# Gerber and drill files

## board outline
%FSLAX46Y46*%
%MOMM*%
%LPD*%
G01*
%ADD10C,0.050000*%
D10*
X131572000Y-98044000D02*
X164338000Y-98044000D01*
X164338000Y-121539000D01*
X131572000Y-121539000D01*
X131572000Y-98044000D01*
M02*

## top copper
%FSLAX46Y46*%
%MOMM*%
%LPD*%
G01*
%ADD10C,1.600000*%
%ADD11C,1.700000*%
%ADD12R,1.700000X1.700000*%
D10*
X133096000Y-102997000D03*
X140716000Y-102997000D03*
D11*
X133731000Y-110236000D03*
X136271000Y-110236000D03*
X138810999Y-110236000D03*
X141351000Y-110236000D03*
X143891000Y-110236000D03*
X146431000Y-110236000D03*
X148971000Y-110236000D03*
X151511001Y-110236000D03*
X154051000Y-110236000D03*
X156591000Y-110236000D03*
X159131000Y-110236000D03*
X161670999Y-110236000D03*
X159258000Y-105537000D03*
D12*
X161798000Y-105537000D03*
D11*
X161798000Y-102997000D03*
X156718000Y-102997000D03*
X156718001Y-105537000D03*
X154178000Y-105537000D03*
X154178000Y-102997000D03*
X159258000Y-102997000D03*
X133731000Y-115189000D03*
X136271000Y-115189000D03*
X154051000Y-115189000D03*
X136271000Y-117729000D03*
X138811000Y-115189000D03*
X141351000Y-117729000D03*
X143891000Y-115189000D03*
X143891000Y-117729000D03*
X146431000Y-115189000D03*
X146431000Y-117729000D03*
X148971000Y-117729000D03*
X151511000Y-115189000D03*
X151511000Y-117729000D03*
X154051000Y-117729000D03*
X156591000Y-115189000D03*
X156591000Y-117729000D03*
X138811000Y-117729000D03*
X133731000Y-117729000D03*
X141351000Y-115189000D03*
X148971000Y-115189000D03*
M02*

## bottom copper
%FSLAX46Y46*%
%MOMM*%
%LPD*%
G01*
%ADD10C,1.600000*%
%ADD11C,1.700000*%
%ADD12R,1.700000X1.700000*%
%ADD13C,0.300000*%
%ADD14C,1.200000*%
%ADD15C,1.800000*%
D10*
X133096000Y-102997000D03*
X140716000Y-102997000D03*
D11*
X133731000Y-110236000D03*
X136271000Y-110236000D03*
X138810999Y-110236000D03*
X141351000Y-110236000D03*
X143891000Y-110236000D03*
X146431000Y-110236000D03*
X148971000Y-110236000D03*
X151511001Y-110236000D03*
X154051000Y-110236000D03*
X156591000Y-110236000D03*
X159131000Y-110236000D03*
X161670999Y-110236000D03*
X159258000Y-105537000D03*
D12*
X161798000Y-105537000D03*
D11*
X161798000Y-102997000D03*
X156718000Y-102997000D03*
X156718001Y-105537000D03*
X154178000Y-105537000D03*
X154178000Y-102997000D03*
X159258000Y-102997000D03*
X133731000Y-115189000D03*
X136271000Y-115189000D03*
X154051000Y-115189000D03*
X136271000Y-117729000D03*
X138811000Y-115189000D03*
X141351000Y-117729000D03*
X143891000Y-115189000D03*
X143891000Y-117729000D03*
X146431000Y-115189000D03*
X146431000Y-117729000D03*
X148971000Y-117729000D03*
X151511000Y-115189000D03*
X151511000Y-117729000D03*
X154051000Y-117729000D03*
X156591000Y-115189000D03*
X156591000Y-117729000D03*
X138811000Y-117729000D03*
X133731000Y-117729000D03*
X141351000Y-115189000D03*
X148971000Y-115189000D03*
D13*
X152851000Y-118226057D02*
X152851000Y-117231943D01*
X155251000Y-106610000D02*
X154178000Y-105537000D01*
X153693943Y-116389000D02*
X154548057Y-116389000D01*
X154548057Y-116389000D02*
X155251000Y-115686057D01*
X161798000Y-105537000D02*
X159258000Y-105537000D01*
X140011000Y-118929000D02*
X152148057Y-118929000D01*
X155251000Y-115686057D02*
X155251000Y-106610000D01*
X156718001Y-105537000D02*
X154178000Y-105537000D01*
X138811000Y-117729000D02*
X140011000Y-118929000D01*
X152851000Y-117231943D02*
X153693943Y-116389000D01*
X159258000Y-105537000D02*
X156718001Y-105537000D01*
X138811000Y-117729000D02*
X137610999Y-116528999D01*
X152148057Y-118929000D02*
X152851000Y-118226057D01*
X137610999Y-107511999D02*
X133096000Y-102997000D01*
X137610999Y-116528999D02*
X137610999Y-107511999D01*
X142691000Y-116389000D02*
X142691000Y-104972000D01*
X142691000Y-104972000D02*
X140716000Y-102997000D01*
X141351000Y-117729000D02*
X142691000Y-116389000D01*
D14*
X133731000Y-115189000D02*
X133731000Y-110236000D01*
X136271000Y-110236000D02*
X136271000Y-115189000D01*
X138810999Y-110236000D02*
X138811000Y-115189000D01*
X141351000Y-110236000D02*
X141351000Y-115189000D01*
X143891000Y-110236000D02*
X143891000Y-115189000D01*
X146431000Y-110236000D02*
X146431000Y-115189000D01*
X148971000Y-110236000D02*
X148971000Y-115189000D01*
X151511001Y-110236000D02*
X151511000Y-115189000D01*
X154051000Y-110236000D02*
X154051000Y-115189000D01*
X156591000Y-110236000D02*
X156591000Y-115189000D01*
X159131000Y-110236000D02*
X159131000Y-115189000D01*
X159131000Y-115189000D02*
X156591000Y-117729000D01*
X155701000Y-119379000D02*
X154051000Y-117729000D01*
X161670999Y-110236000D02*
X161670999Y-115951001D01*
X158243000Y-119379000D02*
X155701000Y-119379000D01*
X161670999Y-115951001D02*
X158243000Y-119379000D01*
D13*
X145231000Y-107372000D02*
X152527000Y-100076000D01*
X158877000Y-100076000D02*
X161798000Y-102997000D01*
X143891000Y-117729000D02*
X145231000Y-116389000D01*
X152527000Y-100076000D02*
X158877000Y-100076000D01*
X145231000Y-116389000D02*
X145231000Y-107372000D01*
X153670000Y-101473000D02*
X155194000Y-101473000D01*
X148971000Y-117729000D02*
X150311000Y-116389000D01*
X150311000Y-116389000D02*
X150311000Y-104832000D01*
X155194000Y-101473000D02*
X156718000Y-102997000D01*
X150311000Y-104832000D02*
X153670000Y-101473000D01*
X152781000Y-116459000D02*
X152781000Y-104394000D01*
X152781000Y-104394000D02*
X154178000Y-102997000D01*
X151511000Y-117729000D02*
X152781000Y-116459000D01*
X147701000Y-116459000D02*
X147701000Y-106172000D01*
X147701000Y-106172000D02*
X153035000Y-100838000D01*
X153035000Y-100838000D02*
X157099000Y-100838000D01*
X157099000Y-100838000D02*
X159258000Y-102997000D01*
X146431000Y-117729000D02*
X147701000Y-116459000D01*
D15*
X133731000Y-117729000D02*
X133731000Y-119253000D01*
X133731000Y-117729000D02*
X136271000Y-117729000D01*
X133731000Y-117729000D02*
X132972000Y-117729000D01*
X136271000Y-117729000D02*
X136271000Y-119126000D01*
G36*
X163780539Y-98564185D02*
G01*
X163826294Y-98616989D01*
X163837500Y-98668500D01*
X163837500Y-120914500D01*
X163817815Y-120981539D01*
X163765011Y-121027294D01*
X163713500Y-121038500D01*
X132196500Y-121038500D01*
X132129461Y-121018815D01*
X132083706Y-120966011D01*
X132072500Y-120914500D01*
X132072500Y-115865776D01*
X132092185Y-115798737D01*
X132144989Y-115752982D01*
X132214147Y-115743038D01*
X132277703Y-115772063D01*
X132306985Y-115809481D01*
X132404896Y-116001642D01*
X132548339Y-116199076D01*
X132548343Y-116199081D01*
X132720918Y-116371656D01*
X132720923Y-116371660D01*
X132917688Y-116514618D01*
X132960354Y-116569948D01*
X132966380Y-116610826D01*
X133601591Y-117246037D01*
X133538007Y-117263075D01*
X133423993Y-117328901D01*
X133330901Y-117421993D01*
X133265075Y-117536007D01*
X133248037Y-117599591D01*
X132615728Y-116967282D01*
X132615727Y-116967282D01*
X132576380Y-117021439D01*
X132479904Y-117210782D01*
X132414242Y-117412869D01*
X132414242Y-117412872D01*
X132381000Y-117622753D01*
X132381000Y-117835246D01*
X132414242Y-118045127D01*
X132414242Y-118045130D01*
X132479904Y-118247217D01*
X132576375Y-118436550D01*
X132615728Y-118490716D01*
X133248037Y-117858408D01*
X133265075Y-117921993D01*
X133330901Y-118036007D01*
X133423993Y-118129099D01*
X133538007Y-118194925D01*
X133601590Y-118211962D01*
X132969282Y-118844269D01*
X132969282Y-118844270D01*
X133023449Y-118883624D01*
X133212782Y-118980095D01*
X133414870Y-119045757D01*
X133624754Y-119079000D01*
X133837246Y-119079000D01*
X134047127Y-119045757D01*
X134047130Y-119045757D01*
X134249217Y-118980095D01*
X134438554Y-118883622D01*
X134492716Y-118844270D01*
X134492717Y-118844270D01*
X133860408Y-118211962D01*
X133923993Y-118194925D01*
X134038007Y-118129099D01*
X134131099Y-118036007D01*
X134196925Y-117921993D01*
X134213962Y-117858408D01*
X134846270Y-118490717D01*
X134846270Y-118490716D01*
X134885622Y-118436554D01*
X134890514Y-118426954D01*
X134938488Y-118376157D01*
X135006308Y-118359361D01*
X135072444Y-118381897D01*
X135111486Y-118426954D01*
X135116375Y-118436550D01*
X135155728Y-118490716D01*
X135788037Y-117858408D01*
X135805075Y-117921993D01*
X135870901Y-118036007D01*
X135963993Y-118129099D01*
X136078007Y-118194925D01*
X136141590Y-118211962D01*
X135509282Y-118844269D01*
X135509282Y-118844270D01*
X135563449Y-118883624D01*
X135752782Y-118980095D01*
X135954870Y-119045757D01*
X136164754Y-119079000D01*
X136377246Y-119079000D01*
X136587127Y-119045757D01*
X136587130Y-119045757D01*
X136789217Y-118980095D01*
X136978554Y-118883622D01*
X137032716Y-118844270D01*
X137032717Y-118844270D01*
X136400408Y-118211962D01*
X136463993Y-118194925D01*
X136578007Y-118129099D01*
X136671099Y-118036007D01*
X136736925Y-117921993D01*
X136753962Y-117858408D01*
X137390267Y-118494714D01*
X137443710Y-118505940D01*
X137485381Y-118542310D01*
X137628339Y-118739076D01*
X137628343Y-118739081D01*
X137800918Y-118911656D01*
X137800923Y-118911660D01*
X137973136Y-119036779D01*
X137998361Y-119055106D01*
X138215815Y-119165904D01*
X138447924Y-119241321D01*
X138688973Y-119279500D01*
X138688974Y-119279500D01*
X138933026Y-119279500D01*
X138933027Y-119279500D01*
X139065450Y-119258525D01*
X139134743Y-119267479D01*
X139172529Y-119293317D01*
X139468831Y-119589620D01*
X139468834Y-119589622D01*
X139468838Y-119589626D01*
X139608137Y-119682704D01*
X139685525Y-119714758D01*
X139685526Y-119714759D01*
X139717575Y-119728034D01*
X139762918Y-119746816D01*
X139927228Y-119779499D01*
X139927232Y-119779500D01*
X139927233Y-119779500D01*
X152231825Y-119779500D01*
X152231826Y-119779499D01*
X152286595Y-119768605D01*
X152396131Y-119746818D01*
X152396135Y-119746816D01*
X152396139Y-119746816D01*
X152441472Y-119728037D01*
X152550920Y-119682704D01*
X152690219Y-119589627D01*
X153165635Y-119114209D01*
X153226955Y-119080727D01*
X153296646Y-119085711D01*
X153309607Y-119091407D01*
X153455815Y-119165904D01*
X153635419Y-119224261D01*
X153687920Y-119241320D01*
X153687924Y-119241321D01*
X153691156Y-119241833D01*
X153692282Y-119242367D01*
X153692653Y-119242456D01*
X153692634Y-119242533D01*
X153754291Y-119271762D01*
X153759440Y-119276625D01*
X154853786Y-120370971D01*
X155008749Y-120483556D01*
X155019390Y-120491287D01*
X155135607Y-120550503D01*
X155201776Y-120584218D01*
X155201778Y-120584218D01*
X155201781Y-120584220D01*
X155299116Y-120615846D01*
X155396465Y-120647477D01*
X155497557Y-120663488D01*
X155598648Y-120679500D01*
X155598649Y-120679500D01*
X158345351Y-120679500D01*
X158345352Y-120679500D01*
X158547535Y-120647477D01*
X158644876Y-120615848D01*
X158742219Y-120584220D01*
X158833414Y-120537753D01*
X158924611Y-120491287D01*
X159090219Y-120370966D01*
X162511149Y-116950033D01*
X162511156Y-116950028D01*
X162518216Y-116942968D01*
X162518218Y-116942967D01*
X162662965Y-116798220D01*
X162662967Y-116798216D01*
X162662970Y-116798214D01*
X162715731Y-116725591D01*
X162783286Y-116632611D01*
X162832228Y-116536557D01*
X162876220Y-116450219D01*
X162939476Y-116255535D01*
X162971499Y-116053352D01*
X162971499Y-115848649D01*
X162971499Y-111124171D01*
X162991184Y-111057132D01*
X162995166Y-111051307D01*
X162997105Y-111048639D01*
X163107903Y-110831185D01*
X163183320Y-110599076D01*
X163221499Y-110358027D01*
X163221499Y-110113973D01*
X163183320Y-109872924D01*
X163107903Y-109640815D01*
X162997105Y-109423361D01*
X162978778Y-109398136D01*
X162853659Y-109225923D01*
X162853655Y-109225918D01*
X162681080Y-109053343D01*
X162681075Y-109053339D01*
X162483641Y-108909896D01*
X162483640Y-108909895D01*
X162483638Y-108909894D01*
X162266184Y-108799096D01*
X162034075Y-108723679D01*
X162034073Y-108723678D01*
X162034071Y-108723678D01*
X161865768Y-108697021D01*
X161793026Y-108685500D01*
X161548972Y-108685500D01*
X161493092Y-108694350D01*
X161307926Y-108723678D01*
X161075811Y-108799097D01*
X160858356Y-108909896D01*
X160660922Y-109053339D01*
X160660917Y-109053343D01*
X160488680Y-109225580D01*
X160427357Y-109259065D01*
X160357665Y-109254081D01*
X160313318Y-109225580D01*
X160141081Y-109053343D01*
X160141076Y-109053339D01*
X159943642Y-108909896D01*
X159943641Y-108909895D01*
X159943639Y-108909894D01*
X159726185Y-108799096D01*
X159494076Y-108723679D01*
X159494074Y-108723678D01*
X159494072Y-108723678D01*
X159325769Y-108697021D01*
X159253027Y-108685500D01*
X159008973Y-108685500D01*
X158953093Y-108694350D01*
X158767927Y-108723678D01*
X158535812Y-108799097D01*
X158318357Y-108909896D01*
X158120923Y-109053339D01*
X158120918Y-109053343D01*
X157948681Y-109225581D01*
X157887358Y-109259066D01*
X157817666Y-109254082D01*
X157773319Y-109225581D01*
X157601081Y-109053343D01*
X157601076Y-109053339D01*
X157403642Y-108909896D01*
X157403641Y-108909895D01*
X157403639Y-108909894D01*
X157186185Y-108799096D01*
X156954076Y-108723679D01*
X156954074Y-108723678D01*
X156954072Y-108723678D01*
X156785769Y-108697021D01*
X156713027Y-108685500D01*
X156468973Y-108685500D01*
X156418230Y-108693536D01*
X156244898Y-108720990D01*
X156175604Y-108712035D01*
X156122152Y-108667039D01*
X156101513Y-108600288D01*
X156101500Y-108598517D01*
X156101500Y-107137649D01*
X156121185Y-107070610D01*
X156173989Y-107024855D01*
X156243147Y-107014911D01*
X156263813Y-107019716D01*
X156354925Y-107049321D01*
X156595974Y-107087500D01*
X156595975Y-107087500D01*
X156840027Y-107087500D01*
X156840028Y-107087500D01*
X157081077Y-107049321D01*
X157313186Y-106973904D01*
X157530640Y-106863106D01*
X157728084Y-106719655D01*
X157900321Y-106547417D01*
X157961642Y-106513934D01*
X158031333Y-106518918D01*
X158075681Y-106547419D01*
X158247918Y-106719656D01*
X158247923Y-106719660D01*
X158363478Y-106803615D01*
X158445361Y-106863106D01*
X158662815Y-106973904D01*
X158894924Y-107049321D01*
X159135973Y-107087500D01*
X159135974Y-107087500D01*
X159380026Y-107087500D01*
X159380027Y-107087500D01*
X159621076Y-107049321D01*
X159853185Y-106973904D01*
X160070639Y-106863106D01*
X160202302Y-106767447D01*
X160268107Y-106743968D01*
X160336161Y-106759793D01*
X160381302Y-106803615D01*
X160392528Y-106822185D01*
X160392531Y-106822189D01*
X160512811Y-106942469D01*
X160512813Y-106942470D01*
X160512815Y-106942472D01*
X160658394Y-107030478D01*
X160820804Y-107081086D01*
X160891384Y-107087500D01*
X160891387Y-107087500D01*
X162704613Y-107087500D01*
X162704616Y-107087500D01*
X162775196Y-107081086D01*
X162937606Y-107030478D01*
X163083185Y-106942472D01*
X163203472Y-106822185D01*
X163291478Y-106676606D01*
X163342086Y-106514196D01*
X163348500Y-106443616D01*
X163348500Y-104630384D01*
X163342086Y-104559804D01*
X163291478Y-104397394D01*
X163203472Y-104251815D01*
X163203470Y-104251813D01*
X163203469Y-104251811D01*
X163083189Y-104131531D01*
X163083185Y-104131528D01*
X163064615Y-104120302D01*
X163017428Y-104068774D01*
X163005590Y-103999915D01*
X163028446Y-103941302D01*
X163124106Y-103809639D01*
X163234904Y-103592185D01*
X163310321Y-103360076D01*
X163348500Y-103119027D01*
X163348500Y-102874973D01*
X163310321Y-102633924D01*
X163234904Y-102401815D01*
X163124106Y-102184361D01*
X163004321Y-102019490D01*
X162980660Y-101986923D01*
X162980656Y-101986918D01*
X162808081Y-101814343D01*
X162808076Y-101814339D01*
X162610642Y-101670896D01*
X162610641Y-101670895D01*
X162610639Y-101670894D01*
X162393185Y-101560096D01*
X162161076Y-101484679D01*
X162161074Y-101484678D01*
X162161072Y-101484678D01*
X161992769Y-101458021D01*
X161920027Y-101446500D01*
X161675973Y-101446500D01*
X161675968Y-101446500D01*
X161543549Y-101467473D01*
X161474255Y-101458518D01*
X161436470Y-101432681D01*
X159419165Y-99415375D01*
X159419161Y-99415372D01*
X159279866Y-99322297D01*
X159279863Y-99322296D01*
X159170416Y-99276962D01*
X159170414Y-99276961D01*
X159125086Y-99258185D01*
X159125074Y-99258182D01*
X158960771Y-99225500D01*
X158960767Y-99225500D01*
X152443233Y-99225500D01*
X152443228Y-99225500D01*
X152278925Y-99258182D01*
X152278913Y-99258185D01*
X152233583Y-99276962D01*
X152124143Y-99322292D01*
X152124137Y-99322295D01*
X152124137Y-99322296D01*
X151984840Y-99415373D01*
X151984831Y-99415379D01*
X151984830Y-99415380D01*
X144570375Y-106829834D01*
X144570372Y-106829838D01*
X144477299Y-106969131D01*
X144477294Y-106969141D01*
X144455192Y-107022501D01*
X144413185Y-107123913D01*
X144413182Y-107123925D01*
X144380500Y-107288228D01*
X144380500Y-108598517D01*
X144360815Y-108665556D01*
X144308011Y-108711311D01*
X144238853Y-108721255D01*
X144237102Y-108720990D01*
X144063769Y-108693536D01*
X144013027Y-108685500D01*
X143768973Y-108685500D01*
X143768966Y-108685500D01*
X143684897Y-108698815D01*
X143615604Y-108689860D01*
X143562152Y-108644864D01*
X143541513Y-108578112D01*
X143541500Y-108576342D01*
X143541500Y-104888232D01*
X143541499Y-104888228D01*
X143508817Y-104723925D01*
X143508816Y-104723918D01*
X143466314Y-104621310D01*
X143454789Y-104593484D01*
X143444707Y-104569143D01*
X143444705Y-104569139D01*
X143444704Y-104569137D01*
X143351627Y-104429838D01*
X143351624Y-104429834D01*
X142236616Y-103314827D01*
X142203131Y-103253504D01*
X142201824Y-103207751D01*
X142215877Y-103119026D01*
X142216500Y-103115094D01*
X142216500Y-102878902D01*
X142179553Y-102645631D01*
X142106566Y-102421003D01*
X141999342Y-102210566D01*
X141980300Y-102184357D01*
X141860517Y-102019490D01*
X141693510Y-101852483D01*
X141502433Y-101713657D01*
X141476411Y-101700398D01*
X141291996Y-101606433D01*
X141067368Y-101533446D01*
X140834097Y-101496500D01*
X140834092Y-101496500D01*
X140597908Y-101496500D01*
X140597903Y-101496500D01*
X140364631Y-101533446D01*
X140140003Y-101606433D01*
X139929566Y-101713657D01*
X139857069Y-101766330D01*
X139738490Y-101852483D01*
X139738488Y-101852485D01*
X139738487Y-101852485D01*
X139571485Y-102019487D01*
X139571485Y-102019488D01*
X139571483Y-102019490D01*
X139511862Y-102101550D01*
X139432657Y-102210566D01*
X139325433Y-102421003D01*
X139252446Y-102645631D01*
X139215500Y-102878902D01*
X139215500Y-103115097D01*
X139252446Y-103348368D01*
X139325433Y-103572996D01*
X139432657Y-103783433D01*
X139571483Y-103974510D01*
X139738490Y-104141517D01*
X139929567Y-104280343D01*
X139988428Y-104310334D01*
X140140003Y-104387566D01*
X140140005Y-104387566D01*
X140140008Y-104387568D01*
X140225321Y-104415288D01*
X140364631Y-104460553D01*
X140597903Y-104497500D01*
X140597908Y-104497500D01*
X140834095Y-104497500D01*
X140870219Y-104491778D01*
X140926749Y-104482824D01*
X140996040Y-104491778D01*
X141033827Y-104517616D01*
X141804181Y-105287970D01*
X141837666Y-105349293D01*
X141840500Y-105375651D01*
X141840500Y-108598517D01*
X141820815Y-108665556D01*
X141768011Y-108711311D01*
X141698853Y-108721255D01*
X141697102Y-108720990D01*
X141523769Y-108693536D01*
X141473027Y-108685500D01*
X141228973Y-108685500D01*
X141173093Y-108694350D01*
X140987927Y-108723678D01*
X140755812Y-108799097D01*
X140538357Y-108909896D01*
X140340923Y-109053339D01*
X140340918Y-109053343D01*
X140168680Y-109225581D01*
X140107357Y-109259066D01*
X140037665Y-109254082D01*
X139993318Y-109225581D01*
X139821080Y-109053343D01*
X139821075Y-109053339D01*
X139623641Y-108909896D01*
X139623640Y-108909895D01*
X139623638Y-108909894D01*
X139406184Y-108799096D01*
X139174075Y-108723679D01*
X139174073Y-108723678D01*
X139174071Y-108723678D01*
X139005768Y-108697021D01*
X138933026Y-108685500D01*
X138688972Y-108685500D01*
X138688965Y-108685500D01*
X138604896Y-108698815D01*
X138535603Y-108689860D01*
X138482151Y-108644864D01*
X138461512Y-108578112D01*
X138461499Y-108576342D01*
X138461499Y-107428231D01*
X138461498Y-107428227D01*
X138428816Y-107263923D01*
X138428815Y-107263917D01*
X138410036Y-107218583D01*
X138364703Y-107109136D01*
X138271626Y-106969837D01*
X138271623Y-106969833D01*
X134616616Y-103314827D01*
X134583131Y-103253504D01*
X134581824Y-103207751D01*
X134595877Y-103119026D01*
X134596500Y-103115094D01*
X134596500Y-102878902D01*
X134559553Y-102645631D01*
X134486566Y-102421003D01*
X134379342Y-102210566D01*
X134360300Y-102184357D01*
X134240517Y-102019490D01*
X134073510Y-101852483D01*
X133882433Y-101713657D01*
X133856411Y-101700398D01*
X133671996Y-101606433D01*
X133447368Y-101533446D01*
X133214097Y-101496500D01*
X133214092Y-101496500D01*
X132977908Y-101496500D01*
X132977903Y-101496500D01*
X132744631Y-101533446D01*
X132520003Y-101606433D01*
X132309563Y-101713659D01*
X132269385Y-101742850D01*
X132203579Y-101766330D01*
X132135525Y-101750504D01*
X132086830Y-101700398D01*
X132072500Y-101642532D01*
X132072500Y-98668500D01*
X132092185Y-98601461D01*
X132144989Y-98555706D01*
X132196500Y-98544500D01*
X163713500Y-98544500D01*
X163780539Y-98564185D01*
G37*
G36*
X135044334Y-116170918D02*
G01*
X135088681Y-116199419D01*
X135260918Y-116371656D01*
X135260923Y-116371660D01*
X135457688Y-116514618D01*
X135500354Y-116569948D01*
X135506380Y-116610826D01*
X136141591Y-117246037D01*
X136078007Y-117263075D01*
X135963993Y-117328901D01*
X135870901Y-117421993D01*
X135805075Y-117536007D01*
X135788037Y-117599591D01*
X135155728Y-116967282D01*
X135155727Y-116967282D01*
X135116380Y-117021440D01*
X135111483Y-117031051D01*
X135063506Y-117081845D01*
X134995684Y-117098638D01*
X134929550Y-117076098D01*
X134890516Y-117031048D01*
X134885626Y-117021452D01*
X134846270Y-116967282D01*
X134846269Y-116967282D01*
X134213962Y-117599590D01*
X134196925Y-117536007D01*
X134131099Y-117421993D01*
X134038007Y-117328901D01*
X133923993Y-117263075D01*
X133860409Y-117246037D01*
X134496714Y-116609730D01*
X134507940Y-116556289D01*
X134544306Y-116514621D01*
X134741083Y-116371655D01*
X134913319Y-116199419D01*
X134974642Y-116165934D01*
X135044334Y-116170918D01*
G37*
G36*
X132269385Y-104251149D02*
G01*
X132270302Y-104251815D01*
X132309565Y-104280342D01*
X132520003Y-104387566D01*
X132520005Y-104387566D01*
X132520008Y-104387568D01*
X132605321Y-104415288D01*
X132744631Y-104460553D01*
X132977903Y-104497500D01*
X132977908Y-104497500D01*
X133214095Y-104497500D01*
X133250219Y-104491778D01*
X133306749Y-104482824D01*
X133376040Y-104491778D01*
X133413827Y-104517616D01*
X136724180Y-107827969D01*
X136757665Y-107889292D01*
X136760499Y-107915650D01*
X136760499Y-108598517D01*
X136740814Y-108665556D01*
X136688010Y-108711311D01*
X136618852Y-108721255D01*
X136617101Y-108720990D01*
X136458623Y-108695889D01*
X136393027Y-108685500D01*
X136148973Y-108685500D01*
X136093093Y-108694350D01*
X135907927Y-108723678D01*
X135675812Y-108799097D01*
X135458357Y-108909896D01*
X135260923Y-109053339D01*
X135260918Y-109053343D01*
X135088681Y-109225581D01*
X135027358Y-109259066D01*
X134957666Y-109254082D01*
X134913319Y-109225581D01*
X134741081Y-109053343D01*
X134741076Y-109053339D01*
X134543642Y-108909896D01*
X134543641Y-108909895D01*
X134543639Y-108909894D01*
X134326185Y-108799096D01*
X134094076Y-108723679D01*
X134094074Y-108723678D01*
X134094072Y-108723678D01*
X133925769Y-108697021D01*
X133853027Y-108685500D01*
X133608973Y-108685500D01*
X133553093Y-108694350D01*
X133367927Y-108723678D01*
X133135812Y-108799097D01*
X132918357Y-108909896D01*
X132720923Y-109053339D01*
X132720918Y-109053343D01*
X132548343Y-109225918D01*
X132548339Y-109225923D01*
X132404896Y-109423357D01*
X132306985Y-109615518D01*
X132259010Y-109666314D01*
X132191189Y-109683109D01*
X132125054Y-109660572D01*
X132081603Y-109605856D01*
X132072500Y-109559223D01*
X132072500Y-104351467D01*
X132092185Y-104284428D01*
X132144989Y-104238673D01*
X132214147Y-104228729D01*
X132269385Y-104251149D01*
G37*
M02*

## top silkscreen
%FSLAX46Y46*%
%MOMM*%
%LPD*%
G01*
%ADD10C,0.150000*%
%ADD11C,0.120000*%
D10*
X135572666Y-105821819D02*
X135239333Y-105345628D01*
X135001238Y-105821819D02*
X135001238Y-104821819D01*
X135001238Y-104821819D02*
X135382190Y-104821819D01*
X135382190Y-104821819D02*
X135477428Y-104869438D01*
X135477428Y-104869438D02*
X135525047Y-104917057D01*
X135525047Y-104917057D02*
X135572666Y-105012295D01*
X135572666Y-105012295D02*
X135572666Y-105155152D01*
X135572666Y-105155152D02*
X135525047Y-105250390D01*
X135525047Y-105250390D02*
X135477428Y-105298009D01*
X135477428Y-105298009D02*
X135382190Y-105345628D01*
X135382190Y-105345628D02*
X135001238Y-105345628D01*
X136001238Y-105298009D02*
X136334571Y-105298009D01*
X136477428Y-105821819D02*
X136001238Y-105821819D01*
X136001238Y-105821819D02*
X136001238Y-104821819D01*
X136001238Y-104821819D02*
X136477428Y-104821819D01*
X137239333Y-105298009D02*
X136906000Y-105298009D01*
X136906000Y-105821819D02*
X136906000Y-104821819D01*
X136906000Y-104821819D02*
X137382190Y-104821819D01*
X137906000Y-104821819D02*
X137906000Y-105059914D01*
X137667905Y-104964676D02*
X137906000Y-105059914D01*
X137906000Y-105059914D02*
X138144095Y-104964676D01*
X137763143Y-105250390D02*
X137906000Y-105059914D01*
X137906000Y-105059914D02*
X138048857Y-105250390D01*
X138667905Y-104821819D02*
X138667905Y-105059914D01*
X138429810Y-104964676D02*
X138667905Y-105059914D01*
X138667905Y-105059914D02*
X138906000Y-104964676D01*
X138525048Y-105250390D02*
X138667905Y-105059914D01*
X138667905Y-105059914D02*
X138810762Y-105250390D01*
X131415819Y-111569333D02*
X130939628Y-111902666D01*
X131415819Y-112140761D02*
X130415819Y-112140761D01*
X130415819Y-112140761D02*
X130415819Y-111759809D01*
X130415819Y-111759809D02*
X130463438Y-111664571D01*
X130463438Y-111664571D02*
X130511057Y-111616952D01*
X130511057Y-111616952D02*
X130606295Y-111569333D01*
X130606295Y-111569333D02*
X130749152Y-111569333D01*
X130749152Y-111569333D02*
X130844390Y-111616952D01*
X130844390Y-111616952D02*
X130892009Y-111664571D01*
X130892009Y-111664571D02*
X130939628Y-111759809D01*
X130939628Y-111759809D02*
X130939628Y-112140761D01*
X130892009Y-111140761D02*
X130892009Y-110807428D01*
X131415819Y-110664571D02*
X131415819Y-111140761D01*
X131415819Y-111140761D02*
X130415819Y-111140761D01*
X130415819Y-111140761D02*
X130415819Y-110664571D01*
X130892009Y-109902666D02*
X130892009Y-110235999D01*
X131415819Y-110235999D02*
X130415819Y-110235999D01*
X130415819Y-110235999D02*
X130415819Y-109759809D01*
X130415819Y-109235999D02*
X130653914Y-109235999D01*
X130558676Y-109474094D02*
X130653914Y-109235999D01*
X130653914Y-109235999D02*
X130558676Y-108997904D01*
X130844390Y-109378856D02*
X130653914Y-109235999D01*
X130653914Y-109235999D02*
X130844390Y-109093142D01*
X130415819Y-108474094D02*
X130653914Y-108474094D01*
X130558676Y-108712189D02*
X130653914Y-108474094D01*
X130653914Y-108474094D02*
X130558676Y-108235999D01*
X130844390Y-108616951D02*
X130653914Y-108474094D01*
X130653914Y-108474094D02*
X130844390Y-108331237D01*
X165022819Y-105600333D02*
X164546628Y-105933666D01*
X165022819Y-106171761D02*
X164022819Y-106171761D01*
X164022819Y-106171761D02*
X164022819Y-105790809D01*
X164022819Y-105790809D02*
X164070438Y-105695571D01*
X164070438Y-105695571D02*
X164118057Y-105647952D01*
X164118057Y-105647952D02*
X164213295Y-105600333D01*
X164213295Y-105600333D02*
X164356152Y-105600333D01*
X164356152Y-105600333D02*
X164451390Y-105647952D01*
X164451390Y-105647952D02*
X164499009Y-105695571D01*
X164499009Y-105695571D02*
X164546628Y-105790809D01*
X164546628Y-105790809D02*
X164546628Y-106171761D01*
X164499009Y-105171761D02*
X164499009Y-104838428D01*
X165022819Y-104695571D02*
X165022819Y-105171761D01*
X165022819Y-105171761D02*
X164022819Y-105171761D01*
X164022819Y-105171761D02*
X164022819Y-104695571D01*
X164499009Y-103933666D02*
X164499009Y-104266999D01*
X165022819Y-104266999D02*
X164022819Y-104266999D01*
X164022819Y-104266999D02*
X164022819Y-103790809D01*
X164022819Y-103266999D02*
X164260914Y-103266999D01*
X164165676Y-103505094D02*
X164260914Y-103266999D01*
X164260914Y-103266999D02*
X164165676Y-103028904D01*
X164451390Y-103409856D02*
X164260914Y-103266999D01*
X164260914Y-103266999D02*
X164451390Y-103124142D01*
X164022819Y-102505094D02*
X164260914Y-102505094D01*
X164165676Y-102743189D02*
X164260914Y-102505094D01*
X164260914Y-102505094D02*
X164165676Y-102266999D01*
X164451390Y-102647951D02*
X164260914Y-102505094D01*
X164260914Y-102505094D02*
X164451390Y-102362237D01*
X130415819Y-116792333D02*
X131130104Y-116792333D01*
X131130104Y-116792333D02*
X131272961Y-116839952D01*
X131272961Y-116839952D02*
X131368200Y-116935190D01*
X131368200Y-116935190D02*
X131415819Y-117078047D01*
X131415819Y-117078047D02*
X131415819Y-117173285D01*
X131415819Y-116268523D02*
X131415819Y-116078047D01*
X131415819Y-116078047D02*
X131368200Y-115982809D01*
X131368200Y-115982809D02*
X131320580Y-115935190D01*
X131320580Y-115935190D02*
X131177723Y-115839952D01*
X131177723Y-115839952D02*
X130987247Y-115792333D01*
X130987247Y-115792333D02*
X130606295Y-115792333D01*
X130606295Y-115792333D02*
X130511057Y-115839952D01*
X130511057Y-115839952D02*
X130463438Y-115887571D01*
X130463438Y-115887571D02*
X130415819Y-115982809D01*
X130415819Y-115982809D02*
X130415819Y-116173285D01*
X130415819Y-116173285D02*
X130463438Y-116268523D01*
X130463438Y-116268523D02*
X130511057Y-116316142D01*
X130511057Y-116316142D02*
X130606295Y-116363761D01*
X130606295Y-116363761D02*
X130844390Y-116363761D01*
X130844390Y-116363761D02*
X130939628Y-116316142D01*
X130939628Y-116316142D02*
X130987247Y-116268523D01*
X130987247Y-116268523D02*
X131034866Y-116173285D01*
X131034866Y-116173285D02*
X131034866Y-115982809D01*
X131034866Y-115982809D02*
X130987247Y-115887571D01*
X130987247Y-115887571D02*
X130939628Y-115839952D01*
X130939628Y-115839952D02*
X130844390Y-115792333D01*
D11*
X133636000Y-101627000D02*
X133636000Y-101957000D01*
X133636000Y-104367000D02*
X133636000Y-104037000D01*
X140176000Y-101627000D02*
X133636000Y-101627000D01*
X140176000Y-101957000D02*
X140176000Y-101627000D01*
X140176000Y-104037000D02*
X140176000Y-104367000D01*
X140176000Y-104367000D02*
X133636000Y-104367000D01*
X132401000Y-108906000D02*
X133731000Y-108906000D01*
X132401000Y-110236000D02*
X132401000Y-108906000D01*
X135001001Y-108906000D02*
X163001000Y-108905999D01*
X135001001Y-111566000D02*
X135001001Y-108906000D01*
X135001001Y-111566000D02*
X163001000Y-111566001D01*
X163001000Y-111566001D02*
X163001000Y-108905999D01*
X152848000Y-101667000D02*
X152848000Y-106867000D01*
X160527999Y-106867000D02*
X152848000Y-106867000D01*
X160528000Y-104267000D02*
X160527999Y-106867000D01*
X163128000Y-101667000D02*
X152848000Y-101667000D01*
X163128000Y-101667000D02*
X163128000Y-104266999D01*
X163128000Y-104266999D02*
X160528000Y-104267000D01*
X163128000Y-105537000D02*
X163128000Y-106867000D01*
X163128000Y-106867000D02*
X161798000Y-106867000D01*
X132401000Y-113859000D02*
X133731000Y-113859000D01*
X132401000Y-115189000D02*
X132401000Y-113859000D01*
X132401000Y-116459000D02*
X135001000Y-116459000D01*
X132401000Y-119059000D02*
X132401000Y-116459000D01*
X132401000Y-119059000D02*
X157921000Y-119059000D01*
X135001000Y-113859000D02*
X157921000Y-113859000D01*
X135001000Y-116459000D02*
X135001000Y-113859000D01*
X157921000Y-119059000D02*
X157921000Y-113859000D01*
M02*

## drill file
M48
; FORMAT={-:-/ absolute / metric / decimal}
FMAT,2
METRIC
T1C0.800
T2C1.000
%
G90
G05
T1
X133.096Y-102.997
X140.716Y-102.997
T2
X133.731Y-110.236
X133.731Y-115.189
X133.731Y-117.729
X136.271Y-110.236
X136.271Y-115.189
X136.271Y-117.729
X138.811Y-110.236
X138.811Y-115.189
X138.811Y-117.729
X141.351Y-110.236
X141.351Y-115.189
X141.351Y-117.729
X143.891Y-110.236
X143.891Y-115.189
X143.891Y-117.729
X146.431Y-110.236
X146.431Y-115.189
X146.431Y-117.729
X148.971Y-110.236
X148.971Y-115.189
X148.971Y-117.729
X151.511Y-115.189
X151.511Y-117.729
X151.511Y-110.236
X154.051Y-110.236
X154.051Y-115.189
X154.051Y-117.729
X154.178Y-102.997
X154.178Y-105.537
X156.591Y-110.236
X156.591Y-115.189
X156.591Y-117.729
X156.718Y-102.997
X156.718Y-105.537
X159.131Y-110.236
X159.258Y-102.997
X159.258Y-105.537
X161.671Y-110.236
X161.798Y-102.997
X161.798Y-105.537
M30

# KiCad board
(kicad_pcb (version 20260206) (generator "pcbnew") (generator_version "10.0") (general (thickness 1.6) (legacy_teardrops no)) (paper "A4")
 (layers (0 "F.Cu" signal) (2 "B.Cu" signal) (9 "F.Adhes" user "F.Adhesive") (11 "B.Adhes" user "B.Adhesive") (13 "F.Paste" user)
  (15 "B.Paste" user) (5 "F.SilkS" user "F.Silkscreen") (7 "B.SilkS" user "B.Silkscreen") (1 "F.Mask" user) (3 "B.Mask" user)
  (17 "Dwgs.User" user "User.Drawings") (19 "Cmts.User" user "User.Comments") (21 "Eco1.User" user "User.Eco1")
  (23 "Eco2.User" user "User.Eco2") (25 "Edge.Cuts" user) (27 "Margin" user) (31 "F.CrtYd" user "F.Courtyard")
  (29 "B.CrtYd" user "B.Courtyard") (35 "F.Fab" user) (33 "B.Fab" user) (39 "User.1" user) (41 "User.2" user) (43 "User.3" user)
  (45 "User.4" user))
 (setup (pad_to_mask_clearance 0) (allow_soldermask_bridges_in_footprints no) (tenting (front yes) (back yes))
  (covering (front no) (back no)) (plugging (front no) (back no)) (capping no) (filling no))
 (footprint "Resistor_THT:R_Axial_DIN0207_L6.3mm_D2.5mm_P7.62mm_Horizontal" (layer "F.Cu") (at 140.716 102.997 180)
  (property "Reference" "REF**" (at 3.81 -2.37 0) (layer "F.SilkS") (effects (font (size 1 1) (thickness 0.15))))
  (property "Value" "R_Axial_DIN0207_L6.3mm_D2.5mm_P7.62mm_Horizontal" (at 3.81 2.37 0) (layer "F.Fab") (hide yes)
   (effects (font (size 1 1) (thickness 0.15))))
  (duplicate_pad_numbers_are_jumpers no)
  (fp_line (start 7.08 1.37) (end 7.08 1.04) (stroke (width 0.12) (type solid)) (layer "F.SilkS"))
  (fp_line (start 7.08 -1.37) (end 7.08 -1.04) (stroke (width 0.12) (type solid)) (layer "F.SilkS"))
  (fp_line (start 0.54 1.37) (end 7.08 1.37) (stroke (width 0.12) (type solid)) (layer "F.SilkS"))
  (fp_line (start 0.54 1.04) (end 0.54 1.37) (stroke (width 0.12) (type solid)) (layer "F.SilkS"))
  (fp_line (start 0.54 -1.04) (end 0.54 -1.37) (stroke (width 0.12) (type solid)) (layer "F.SilkS"))
  (fp_line (start 0.54 -1.37) (end 7.08 -1.37) (stroke (width 0.12) (type solid)) (layer "F.SilkS"))
  (pad "3" thru_hole circle (at 7.62 0 180) (size 1.6 1.6) (drill 0.8) (layers "*.Cu" "*.Mask") (remove_unused_layers no) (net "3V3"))
  (pad "con" thru_hole circle (at 0 0 180) (size 1.6 1.6) (drill 0.8) (layers "*.Cu" "*.Mask") (remove_unused_layers no) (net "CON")))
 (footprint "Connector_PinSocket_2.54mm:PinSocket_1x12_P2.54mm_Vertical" (layer "F.Cu") (at 133.731 110.236 90)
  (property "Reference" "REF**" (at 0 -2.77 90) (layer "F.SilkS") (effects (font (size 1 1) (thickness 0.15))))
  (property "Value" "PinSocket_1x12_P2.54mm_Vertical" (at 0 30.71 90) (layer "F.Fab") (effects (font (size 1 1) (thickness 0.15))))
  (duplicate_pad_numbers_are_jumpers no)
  (fp_line (start 1.33 -1.33) (end 1.33 0) (stroke (width 0.12) (type solid)) (layer "F.SilkS"))
  (fp_line (start 0 -1.33) (end 1.33 -1.33) (stroke (width 0.12) (type solid)) (layer "F.SilkS"))
  (fp_line (start 1.33 1.270001) (end 1.330001 29.27) (stroke (width 0.12) (type solid)) (layer "F.SilkS"))
  (fp_line (start -1.33 1.270001) (end 1.33 1.270001) (stroke (width 0.12) (type solid)) (layer "F.SilkS"))
  (fp_line (start -1.33 1.270001) (end -1.330001 29.27) (stroke (width 0.12) (type solid)) (layer "F.SilkS"))
  (fp_line (start -1.330001 29.27) (end 1.330001 29.27) (stroke (width 0.12) (type solid)) (layer "F.SilkS"))
  (pad "1" thru_hole circle (at 0 0 90) (size 1.7 1.7) (drill 1) (layers "*.Cu" "*.Mask") (remove_unused_layers no) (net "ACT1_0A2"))
  (pad "2" thru_hole circle (at 0 2.54 90) (size 1.7 1.7) (drill 1) (layers "*.Cu" "*.Mask") (remove_unused_layers no) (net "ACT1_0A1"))
  (pad "3" thru_hole circle (at 0 5.079999 90) (size 1.7 1.7) (drill 1) (layers "*.Cu" "*.Mask") (remove_unused_layers no) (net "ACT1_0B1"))
  (pad "4" thru_hole circle (at 0 7.62 90) (size 1.7 1.7) (drill 1) (layers "*.Cu" "*.Mask") (remove_unused_layers no) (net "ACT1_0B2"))
  (pad "5" thru_hole circle (at 0 10.16 90) (size 1.7 1.7) (drill 1) (layers "*.Cu" "*.Mask") (remove_unused_layers no) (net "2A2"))
  (pad "6" thru_hole circle (at 0 12.7 90) (size 1.7 1.7) (drill 1) (layers "*.Cu" "*.Mask") (remove_unused_layers no) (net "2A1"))
  (pad "7" thru_hole circle (at 0 15.24 90) (size 1.7 1.7) (drill 1) (layers "*.Cu" "*.Mask") (remove_unused_layers no) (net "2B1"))
  (pad "8" thru_hole circle (at 0 17.780001 90) (size 1.7 1.7) (drill 1) (layers "*.Cu" "*.Mask") (remove_unused_layers no) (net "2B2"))
  (pad "9" thru_hole circle (at 0 20.32 90) (size 1.7 1.7) (drill 1) (layers "*.Cu" "*.Mask") (remove_unused_layers no) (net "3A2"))
  (pad "10" thru_hole circle (at 0 22.86 90) (size 1.7 1.7) (drill 1) (layers "*.Cu" "*.Mask") (remove_unused_layers no) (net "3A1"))
  (pad "11" thru_hole circle (at 0 25.4 90) (size 1.7 1.7) (drill 1) (layers "*.Cu" "*.Mask") (remove_unused_layers no) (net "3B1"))
  (pad "12" thru_hole circle (at 0 27.939999 90) (size 1.7 1.7) (drill 1) (layers "*.Cu" "*.Mask") (remove_unused_layers no) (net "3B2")))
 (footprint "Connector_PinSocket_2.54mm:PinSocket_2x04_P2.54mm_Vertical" (layer "F.Cu") (at 161.798 105.537 -90)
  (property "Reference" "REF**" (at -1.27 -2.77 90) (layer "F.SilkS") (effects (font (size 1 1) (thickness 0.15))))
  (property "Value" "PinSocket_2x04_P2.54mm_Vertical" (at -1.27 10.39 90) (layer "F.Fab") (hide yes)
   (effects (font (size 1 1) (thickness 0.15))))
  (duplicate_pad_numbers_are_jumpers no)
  (fp_line (start -3.87 8.95) (end 1.33 8.95) (stroke (width 0.12) (type solid)) (layer "F.SilkS"))
  (fp_line (start 1.33 1.270001) (end 1.33 8.95) (stroke (width 0.12) (type solid)) (layer "F.SilkS"))
  (fp_line (start -1.27 1.27) (end 1.33 1.270001) (stroke (width 0.12) (type solid)) (layer "F.SilkS"))
  (fp_line (start -3.87 -1.33) (end -3.87 8.95) (stroke (width 0.12) (type solid)) (layer "F.SilkS"))
  (fp_line (start -3.87 -1.33) (end -1.270001 -1.33) (stroke (width 0.12) (type solid)) (layer "F.SilkS"))
  (fp_line (start -1.270001 -1.33) (end -1.27 1.27) (stroke (width 0.12) (type solid)) (layer "F.SilkS"))
  (fp_line (start 0 -1.33) (end 1.33 -1.33) (stroke (width 0.12) (type solid)) (layer "F.SilkS"))
  (fp_line (start 1.33 -1.33) (end 1.33 0) (stroke (width 0.12) (type solid)) (layer "F.SilkS"))
  (pad "" thru_hole circle (at 0 2.54 270) (size 1.7 1.7) (drill 1) (layers "*.Cu" "*.Mask") (remove_unused_layers no) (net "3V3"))
  (pad "1" thru_hole rect (at 0 0 270) (size 1.7 1.7) (drill 1) (layers "*.Cu" "*.Mask") (remove_unused_layers no) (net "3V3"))
  (pad "2" thru_hole circle (at -2.54 0 270) (size 1.7 1.7) (drill 1) (layers "*.Cu" "*.Mask") (remove_unused_layers no) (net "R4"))
  (pad "2" thru_hole circle (at -2.54 5.08 270) (size 1.7 1.7) (drill 1) (layers "*.Cu" "*.Mask") (remove_unused_layers no) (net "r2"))
  (pad "5" thru_hole circle (at 0 5.079999 270) (size 1.7 1.7) (drill 1) (layers "*.Cu" "*.Mask") (remove_unused_layers no) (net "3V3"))
  (pad "7" thru_hole circle (at 0 7.62 270) (size 1.7 1.7) (drill 1) (layers "*.Cu" "*.Mask") (remove_unused_layers no) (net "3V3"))
  (pad "8" thru_hole circle (at -2.54 7.62 270) (size 1.7 1.7) (drill 1) (layers "*.Cu" "*.Mask") (remove_unused_layers no) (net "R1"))
  (pad "r" thru_hole circle (at -2.54 2.54 270) (size 1.7 1.7) (drill 1) (layers "*.Cu" "*.Mask") (remove_unused_layers no) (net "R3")))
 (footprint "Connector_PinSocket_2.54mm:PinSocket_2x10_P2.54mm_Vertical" (layer "F.Cu") (at 133.731 115.189 90)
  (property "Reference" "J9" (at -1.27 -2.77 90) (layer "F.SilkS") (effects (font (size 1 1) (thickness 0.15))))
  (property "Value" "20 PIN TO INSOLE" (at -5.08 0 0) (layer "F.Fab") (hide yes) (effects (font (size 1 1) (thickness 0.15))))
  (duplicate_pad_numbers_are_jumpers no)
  (fp_line (start 1.33 -1.33) (end 1.33 0) (stroke (width 0.12) (type solid)) (layer "F.SilkS"))
  (fp_line (start 0 -1.33) (end 1.33 -1.33) (stroke (width 0.12) (type solid)) (layer "F.SilkS"))
  (fp_line (start -1.27 -1.33) (end -1.27 1.27) (stroke (width 0.12) (type solid)) (layer "F.SilkS"))
  (fp_line (start -3.87 -1.33) (end -1.27 -1.33) (stroke (width 0.12) (type solid)) (layer "F.SilkS"))
  (fp_line (start -3.87 -1.33) (end -3.87 24.19) (stroke (width 0.12) (type solid)) (layer "F.SilkS"))
  (fp_line (start 1.33 1.27) (end 1.33 24.19) (stroke (width 0.12) (type solid)) (layer "F.SilkS"))
  (fp_line (start -1.27 1.27) (end 1.33 1.27) (stroke (width 0.12) (type solid)) (layer "F.SilkS"))
  (fp_line (start -3.87 24.19) (end 1.33 24.19) (stroke (width 0.12) (type solid)) (layer "F.SilkS"))
  (pad "1" thru_hole circle (at 0 0 90) (size 1.7 1.7) (drill 1) (layers "*.Cu" "*.Mask") (remove_unused_layers no) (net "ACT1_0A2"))
  (pad "3" thru_hole circle (at 0 2.54 90) (size 1.7 1.7) (drill 1) (layers "*.Cu" "*.Mask") (remove_unused_layers no) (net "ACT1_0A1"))
  (pad "3B2" thru_hole circle (at 0 20.32 90) (size 1.7 1.7) (drill 1) (layers "*.Cu" "*.Mask") (remove_unused_layers no) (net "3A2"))
  (pad "4" thru_hole circle (at -2.54 2.54 90) (size 1.7 1.7) (drill 1) (layers "*.Cu" "*.Mask") (remove_unused_layers no) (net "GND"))
  (pad "5" thru_hole circle (at 0 5.08 90) (size 1.7 1.7) (drill 1) (layers "*.Cu" "*.Mask") (remove_unused_layers no) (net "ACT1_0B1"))
  (pad "8" thru_hole circle (at -2.54 7.62 90) (size 1.7 1.7) (drill 1) (layers "*.Cu" "*.Mask") (remove_unused_layers no) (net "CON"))
  (pad "9" thru_hole circle (at 0 10.16 90) (size 1.7 1.7) (drill 1) (layers "*.Cu" "*.Mask") (remove_unused_layers no) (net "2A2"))
  (pad "10" thru_hole circle (at -2.54 10.16 90) (size 1.7 1.7) (drill 1) (layers "*.Cu" "*.Mask") (remove_unused_layers no) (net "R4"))
  (pad "11" thru_hole circle (at 0 12.7 90) (size 1.7 1.7) (drill 1) (layers "*.Cu" "*.Mask") (remove_unused_layers no) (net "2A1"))
  (pad "12" thru_hole circle (at -2.54 12.7 90) (size 1.7 1.7) (drill 1) (layers "*.Cu" "*.Mask") (remove_unused_layers no) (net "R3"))
  (pad "14" thru_hole circle (at -2.54 15.24 90) (size 1.7 1.7) (drill 1) (layers "*.Cu" "*.Mask") (remove_unused_layers no) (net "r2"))
  (pad "15" thru_hole circle (at 0 17.78 90) (size 1.7 1.7) (drill 1) (layers "*.Cu" "*.Mask") (remove_unused_layers no) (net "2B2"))
  (pad "16" thru_hole circle (at -2.54 17.78 90) (size 1.7 1.7) (drill 1) (layers "*.Cu" "*.Mask") (remove_unused_layers no) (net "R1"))
  (pad "18" thru_hole circle (at -2.54 20.32 90) (size 1.7 1.7) (drill 1) (layers "*.Cu" "*.Mask") (remove_unused_layers no) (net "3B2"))
  (pad "19" thru_hole circle (at 0 22.86 90) (size 1.7 1.7) (drill 1) (layers "*.Cu" "*.Mask") (remove_unused_layers no) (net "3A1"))
  (pad "20" thru_hole circle (at -2.54 22.86 90) (size 1.7 1.7) (drill 1) (layers "*.Cu" "*.Mask") (remove_unused_layers no) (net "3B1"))
  (pad "A" thru_hole circle (at -2.54 5.08 90) (size 1.7 1.7) (drill 1) (layers "*.Cu" "*.Mask") (remove_unused_layers no) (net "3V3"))
  (pad "ACT1_0A2" thru_hole circle (at -2.54 0 90) (size 1.7 1.7) (drill 1) (layers "*.Cu" "*.Mask") (remove_unused_layers no) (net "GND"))
  (pad "CON" thru_hole circle (at 0 7.62 90) (size 1.7 1.7) (drill 1) (layers "*.Cu" "*.Mask" "Dwgs.User") (remove_unused_layers no)
   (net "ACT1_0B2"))
  (pad "R2" thru_hole circle (at 0 15.24 90) (size 1.7 1.7) (drill 1) (layers "*.Cu" "F.Mask") (remove_unused_layers no) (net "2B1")))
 (gr_rect (start 131.572 98.044) (end 164.338 121.539) (stroke (width 0.05) (type default)) (fill no) (layer "Edge.Cuts"))
 (segment (start 152.851 118.226057) (end 152.851 117.231943) (width 0.3) (layer "B.Cu") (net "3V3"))
 (segment (start 155.251 106.61) (end 154.178 105.537) (width 0.3) (layer "B.Cu") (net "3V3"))
 (segment (start 153.693943 116.389) (end 154.548057 116.389) (width 0.3) (layer "B.Cu") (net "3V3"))
 (segment (start 154.548057 116.389) (end 155.251 115.686057) (width 0.3) (layer "B.Cu") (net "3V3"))
 (segment (start 161.798 105.537) (end 159.258 105.537) (width 0.3) (layer "B.Cu") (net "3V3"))
 (segment (start 140.011 118.929) (end 152.148057 118.929) (width 0.3) (layer "B.Cu") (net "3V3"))
 (segment (start 155.251 115.686057) (end 155.251 106.61) (width 0.3) (layer "B.Cu") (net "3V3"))
 (segment (start 156.718001 105.537) (end 154.178 105.537) (width 0.3) (layer "B.Cu") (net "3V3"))
 (segment (start 138.811 117.729) (end 140.011 118.929) (width 0.3) (layer "B.Cu") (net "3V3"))
 (segment (start 152.851 117.231943) (end 153.693943 116.389) (width 0.3) (layer "B.Cu") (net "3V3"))
 (segment (start 159.258 105.537) (end 156.718001 105.537) (width 0.3) (layer "B.Cu") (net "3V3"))
 (segment (start 138.811 117.729) (end 137.610999 116.528999) (width 0.3) (layer "B.Cu") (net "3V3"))
 (segment (start 152.148057 118.929) (end 152.851 118.226057) (width 0.3) (layer "B.Cu") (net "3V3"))
 (segment (start 137.610999 107.511999) (end 133.096 102.997) (width 0.3) (layer "B.Cu") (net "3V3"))
 (segment (start 137.610999 116.528999) (end 137.610999 107.511999) (width 0.3) (layer "B.Cu") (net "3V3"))
 (segment (start 142.691 116.389) (end 142.691 104.972) (width 0.3) (layer "B.Cu") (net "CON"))
 (segment (start 142.691 104.972) (end 140.716 102.997) (width 0.3) (layer "B.Cu") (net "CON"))
 (segment (start 141.351 117.729) (end 142.691 116.389) (width 0.3) (layer "B.Cu") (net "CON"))
 (segment (start 133.731 115.189) (end 133.731 110.236) (width 1.2) (layer "B.Cu") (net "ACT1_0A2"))
 (segment (start 136.271 110.236) (end 136.271 115.189) (width 1.2) (layer "B.Cu") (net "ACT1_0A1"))
 (segment (start 138.810999 110.236) (end 138.811 115.189) (width 1.2) (layer "B.Cu") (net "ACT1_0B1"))
 (segment (start 141.351 110.236) (end 141.351 115.189) (width 1.2) (layer "B.Cu") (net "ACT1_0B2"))
 (segment (start 143.891 110.236) (end 143.891 115.189) (width 1.2) (layer "B.Cu") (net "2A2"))
 (segment (start 146.431 110.236) (end 146.431 115.189) (width 1.2) (layer "B.Cu") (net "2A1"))
 (segment (start 148.971 110.236) (end 148.971 115.189) (width 1.2) (layer "B.Cu") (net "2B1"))
 (segment (start 151.511001 110.236) (end 151.511 115.189) (width 1.2) (layer "B.Cu") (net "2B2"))
 (segment (start 154.051 110.236) (end 154.051 115.189) (width 1.2) (layer "B.Cu") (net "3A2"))
 (segment (start 156.591 110.236) (end 156.591 115.189) (width 1.2) (layer "B.Cu") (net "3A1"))
 (segment (start 159.131 110.236) (end 159.131 115.189) (width 1.2) (layer "B.Cu") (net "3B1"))
 (segment (start 159.131 115.189) (end 156.591 117.729) (width 1.2) (layer "B.Cu") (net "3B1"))
 (segment (start 155.701 119.379) (end 154.051 117.729) (width 1.2) (layer "B.Cu") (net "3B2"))
 (segment (start 161.670999 110.236) (end 161.670999 115.951001) (width 1.2) (layer "B.Cu") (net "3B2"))
 (segment (start 158.243 119.379) (end 155.701 119.379) (width 1.2) (layer "B.Cu") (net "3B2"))
 (segment (start 161.670999 115.951001) (end 158.243 119.379) (width 1.2) (layer "B.Cu") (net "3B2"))
 (segment (start 145.231 107.372) (end 152.527 100.076) (width 0.3) (layer "B.Cu") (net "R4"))
 (segment (start 158.877 100.076) (end 161.798 102.997) (width 0.3) (layer "B.Cu") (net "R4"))
 (segment (start 143.891 117.729) (end 145.231 116.389) (width 0.3) (layer "B.Cu") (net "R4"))
 (segment (start 152.527 100.076) (end 158.877 100.076) (width 0.3) (layer "B.Cu") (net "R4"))
 (segment (start 145.231 116.389) (end 145.231 107.372) (width 0.3) (layer "B.Cu") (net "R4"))
 (segment (start 153.67 101.473) (end 155.194 101.473) (width 0.3) (layer "B.Cu") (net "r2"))
 (segment (start 148.971 117.729) (end 150.311 116.389) (width 0.3) (layer "B.Cu") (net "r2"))
 (segment (start 150.311 116.389) (end 150.311 104.832) (width 0.3) (layer "B.Cu") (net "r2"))
 (segment (start 155.194 101.473) (end 156.718 102.997) (width 0.3) (layer "B.Cu") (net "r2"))
 (segment (start 150.311 104.832) (end 153.67 101.473) (width 0.3) (layer "B.Cu") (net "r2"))
 (segment (start 152.781 116.459) (end 152.781 104.394) (width 0.3) (layer "B.Cu") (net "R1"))
 (segment (start 152.781 104.394) (end 154.178 102.997) (width 0.3) (layer "B.Cu") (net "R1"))
 (segment (start 151.511 117.729) (end 152.781 116.459) (width 0.3) (layer "B.Cu") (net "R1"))
 (segment (start 147.701 116.459) (end 147.701 106.172) (width 0.3) (layer "B.Cu") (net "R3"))
 (segment (start 147.701 106.172) (end 153.035 100.838) (width 0.3) (layer "B.Cu") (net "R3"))
 (segment (start 153.035 100.838) (end 157.099 100.838) (width 0.3) (layer "B.Cu") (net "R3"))
 (segment (start 157.099 100.838) (end 159.258 102.997) (width 0.3) (layer "B.Cu") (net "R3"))
 (segment (start 146.431 117.729) (end 147.701 116.459) (width 0.3) (layer "B.Cu") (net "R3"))
 (segment (start 133.731 117.729) (end 133.731 119.253) (width 1.8) (layer "B.Cu") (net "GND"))
 (segment (start 133.731 117.729) (end 136.271 117.729) (width 1.8) (layer "B.Cu") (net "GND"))
 (segment (start 133.731 117.729) (end 132.972 117.729) (width 1.8) (layer "B.Cu") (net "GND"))
 (segment (start 136.271 117.729) (end 136.271 119.126) (width 1.8) (layer "B.Cu") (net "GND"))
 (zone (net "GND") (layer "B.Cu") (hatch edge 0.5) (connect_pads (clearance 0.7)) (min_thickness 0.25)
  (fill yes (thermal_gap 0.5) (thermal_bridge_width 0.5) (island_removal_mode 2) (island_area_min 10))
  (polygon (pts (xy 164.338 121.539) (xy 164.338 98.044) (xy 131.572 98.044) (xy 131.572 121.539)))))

